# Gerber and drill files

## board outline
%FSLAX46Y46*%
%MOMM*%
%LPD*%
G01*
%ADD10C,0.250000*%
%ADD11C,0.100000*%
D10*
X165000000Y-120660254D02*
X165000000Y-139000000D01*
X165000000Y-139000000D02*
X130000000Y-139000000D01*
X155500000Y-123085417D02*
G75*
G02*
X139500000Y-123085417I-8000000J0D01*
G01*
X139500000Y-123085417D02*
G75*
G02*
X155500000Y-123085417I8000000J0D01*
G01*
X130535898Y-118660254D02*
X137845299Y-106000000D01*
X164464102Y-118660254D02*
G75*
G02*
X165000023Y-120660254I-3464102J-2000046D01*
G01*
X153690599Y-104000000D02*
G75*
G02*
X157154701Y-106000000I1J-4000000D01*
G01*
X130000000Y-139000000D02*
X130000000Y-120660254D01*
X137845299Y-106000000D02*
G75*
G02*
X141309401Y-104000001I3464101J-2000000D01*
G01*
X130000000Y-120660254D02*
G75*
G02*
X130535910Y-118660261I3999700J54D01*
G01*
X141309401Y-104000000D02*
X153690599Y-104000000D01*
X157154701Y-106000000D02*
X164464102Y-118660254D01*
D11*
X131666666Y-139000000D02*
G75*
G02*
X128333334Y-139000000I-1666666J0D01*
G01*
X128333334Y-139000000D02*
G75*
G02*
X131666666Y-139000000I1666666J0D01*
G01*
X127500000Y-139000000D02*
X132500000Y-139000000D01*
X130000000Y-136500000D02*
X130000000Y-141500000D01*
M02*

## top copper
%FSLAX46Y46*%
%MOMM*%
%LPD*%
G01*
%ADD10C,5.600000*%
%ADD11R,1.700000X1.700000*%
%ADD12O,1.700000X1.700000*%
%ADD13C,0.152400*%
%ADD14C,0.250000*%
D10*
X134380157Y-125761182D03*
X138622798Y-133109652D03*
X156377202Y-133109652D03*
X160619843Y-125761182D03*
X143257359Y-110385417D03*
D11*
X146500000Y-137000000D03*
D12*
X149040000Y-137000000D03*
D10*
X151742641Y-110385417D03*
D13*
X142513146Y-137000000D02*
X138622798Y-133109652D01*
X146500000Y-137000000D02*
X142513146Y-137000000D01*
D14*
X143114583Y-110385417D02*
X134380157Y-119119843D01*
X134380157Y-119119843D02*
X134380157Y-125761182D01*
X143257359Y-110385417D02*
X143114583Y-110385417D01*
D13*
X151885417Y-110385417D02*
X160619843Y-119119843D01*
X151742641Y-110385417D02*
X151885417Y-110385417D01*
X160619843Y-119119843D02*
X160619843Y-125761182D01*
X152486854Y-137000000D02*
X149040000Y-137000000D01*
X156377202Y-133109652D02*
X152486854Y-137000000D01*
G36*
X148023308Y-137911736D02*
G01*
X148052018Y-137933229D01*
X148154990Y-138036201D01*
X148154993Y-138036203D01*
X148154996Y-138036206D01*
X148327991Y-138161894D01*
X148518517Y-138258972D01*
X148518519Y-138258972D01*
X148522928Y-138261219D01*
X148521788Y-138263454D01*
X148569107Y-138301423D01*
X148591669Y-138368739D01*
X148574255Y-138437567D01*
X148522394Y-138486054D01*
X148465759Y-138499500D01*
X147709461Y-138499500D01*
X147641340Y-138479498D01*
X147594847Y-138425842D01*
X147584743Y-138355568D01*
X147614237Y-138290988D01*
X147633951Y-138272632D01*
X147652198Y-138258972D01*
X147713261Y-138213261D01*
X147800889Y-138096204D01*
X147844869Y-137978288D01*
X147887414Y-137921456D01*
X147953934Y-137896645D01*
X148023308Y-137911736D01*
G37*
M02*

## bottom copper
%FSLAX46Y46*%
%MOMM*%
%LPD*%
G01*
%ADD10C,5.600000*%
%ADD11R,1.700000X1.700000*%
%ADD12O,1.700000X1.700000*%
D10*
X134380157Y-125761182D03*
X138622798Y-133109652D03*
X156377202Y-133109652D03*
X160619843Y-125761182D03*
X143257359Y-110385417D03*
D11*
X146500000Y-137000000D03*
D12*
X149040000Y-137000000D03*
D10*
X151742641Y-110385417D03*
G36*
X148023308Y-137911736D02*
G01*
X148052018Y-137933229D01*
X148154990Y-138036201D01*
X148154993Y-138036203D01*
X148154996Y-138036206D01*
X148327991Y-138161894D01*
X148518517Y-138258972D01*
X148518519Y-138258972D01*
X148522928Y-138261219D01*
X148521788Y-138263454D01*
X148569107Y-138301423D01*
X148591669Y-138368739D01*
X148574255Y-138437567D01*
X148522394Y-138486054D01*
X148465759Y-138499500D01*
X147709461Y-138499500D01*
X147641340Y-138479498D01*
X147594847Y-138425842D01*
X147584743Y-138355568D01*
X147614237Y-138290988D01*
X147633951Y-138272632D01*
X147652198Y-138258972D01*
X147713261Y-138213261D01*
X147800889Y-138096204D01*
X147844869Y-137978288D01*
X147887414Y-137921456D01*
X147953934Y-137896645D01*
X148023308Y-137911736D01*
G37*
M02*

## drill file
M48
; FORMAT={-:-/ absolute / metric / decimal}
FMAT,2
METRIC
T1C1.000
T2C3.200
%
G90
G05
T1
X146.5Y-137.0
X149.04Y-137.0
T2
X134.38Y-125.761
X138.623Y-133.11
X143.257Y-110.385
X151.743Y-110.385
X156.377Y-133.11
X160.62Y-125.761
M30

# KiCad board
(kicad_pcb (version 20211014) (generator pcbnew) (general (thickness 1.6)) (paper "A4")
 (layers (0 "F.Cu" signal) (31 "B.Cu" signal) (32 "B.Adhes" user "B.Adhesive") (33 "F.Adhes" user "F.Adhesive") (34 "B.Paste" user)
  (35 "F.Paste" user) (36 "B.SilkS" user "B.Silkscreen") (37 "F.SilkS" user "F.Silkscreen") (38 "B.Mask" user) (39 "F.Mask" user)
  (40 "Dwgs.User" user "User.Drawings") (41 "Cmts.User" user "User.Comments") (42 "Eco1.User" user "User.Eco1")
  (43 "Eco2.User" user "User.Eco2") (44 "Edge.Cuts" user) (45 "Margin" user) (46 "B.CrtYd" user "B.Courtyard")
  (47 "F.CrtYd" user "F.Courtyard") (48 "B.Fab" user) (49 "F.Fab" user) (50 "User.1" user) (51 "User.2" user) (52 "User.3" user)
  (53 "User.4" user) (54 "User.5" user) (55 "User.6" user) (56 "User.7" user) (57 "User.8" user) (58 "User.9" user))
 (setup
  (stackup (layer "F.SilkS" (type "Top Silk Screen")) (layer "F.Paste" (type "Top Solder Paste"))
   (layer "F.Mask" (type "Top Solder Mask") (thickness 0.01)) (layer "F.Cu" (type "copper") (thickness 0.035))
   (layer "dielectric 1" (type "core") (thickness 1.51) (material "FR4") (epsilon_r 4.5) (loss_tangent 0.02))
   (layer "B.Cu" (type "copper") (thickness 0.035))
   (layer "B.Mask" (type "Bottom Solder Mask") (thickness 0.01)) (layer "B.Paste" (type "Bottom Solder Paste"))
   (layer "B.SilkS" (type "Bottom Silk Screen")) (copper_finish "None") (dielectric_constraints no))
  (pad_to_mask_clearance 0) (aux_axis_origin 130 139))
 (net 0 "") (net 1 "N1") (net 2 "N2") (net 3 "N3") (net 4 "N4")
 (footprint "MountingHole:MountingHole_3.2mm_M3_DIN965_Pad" (layer "F.Cu") (at 134.380157 125.761182)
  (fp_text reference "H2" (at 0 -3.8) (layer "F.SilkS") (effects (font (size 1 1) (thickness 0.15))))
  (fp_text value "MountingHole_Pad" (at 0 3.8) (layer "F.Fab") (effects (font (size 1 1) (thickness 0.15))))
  (pad "1" thru_hole circle (at 0 0) (size 5.6 5.6) (drill 3.2) (layers *.Cu *.Mask) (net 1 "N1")))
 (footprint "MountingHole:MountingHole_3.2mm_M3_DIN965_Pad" (layer "F.Cu") (at 138.622798 133.109652)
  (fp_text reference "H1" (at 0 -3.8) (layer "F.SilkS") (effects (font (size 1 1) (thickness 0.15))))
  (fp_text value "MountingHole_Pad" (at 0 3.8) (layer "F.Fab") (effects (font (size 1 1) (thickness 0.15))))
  (pad "1" thru_hole circle (at 0 0) (size 5.6 5.6) (drill 3.2) (layers *.Cu *.Mask) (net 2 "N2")))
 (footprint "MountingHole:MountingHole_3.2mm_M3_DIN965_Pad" (layer "F.Cu") (at 156.377202 133.109652)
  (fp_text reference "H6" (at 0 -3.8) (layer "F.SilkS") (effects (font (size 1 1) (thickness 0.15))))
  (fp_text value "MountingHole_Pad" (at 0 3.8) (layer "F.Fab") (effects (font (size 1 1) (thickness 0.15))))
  (pad "1" thru_hole circle (at 0 0) (size 5.6 5.6) (drill 3.2) (layers *.Cu *.Mask) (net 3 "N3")))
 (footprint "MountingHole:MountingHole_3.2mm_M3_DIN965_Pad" (layer "F.Cu") (at 160.619843 125.761182)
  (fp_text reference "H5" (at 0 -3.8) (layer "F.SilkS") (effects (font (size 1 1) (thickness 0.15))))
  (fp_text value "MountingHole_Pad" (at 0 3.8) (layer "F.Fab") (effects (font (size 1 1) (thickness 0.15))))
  (pad "1" thru_hole circle (at 0 0) (size 5.6 5.6) (drill 3.2) (layers *.Cu *.Mask) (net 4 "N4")))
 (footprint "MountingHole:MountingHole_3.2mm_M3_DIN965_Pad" (layer "F.Cu") (at 143.257359 110.385417)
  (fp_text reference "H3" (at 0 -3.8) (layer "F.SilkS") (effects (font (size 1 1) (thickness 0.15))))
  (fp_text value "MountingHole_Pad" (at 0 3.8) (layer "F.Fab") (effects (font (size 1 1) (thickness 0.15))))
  (pad "1" thru_hole circle (at 0 0) (size 5.6 5.6) (drill 3.2) (layers *.Cu *.Mask) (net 1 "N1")))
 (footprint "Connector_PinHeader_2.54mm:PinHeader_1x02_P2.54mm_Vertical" (layer "F.Cu") (at 146.5 137 90)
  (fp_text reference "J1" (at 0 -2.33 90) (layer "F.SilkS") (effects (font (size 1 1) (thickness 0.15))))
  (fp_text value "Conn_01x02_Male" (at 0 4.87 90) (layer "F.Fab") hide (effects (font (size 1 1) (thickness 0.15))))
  (pad "1" thru_hole rect (at 0 0 90) (size 1.7 1.7) (drill 1) (layers *.Cu *.Mask) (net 2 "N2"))
  (pad "2" thru_hole oval (at 0 2.54 90) (size 1.7 1.7) (drill 1) (layers *.Cu *.Mask) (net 3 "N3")))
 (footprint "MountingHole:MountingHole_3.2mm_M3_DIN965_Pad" (layer "F.Cu") (at 151.742641 110.385417)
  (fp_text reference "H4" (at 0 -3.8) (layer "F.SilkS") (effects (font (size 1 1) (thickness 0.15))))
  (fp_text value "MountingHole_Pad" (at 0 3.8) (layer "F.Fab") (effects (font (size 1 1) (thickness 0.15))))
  (pad "1" thru_hole circle (at 0 0) (size 5.6 5.6) (drill 3.2) (layers *.Cu *.Mask) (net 4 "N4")))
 (gr_line (start 165 120.660254) (end 165 139) (layer "Edge.Cuts") (width 0.25))
 (gr_line (start 165 139) (end 130 139) (layer "Edge.Cuts") (width 0.25))
 (gr_circle (center 147.5 123.085417) (end 139.5 123.085417) (layer "Edge.Cuts") (width 0.25) (fill none))
 (gr_line (start 130.535898 118.660254) (end 137.845299 106) (layer "Edge.Cuts") (width 0.25))
 (gr_arc (start 164.464102 118.660254) (mid 164.863703 119.624978) (end 165 120.660254) (layer "Edge.Cuts") (width 0.25))
 (gr_arc (start 153.690599 104) (mid 155.690599 104.535898) (end 157.154701 106) (layer "Edge.Cuts") (width 0.25))
 (gr_line (start 130 139) (end 130 120.660254) (layer "Edge.Cuts") (width 0.25))
 (gr_arc (start 137.845299 106) (mid 139.309403 104.535904) (end 141.309401 104) (layer "Edge.Cuts") (width 0.25))
 (gr_arc (start 130 120.660254) (mid 130.136288 119.624974) (end 130.535898 118.660254) (layer "Edge.Cuts") (width 0.25))
 (gr_line (start 141.309401 104) (end 153.690599 104) (layer "Edge.Cuts") (width 0.25))
 (gr_line (start 157.154701 106) (end 164.464102 118.660254) (layer "Edge.Cuts") (width 0.25))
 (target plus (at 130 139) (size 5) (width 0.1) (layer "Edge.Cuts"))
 (segment (start 142.513146 137) (end 138.622798 133.109652) (width 0.1524) (layer "F.Cu") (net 2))
 (segment (start 146.5 137) (end 142.513146 137) (width 0.1524) (layer "F.Cu") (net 2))
 (segment (start 143.114583 110.385417) (end 134.380157 119.119843) (width 0.25) (layer "F.Cu") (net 1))
 (segment (start 134.380157 119.119843) (end 134.380157 125.761182) (width 0.25) (layer "F.Cu") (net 1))
 (segment (start 143.257359 110.385417) (end 143.114583 110.385417) (width 0.25) (layer "F.Cu") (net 1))
 (segment (start 151.885417 110.385417) (end 160.619843 119.119843) (width 0.1524) (layer "F.Cu") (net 4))
 (segment (start 151.742641 110.385417) (end 151.885417 110.385417) (width 0.1524) (layer "F.Cu") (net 4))
 (segment (start 160.619843 119.119843) (end 160.619843 125.761182) (width 0.1524) (layer "F.Cu") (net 4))
 (segment (start 152.486854 137) (end 149.04 137) (width 0.1524) (layer "F.Cu") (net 3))
 (segment (start 156.377202 133.109652) (end 152.486854 137) (width 0.1524) (layer "F.Cu") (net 3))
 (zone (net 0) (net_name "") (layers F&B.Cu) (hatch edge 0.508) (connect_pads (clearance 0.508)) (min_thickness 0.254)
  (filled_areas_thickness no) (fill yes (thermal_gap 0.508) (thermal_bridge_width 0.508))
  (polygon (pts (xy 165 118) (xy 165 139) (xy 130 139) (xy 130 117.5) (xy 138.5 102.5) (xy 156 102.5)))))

